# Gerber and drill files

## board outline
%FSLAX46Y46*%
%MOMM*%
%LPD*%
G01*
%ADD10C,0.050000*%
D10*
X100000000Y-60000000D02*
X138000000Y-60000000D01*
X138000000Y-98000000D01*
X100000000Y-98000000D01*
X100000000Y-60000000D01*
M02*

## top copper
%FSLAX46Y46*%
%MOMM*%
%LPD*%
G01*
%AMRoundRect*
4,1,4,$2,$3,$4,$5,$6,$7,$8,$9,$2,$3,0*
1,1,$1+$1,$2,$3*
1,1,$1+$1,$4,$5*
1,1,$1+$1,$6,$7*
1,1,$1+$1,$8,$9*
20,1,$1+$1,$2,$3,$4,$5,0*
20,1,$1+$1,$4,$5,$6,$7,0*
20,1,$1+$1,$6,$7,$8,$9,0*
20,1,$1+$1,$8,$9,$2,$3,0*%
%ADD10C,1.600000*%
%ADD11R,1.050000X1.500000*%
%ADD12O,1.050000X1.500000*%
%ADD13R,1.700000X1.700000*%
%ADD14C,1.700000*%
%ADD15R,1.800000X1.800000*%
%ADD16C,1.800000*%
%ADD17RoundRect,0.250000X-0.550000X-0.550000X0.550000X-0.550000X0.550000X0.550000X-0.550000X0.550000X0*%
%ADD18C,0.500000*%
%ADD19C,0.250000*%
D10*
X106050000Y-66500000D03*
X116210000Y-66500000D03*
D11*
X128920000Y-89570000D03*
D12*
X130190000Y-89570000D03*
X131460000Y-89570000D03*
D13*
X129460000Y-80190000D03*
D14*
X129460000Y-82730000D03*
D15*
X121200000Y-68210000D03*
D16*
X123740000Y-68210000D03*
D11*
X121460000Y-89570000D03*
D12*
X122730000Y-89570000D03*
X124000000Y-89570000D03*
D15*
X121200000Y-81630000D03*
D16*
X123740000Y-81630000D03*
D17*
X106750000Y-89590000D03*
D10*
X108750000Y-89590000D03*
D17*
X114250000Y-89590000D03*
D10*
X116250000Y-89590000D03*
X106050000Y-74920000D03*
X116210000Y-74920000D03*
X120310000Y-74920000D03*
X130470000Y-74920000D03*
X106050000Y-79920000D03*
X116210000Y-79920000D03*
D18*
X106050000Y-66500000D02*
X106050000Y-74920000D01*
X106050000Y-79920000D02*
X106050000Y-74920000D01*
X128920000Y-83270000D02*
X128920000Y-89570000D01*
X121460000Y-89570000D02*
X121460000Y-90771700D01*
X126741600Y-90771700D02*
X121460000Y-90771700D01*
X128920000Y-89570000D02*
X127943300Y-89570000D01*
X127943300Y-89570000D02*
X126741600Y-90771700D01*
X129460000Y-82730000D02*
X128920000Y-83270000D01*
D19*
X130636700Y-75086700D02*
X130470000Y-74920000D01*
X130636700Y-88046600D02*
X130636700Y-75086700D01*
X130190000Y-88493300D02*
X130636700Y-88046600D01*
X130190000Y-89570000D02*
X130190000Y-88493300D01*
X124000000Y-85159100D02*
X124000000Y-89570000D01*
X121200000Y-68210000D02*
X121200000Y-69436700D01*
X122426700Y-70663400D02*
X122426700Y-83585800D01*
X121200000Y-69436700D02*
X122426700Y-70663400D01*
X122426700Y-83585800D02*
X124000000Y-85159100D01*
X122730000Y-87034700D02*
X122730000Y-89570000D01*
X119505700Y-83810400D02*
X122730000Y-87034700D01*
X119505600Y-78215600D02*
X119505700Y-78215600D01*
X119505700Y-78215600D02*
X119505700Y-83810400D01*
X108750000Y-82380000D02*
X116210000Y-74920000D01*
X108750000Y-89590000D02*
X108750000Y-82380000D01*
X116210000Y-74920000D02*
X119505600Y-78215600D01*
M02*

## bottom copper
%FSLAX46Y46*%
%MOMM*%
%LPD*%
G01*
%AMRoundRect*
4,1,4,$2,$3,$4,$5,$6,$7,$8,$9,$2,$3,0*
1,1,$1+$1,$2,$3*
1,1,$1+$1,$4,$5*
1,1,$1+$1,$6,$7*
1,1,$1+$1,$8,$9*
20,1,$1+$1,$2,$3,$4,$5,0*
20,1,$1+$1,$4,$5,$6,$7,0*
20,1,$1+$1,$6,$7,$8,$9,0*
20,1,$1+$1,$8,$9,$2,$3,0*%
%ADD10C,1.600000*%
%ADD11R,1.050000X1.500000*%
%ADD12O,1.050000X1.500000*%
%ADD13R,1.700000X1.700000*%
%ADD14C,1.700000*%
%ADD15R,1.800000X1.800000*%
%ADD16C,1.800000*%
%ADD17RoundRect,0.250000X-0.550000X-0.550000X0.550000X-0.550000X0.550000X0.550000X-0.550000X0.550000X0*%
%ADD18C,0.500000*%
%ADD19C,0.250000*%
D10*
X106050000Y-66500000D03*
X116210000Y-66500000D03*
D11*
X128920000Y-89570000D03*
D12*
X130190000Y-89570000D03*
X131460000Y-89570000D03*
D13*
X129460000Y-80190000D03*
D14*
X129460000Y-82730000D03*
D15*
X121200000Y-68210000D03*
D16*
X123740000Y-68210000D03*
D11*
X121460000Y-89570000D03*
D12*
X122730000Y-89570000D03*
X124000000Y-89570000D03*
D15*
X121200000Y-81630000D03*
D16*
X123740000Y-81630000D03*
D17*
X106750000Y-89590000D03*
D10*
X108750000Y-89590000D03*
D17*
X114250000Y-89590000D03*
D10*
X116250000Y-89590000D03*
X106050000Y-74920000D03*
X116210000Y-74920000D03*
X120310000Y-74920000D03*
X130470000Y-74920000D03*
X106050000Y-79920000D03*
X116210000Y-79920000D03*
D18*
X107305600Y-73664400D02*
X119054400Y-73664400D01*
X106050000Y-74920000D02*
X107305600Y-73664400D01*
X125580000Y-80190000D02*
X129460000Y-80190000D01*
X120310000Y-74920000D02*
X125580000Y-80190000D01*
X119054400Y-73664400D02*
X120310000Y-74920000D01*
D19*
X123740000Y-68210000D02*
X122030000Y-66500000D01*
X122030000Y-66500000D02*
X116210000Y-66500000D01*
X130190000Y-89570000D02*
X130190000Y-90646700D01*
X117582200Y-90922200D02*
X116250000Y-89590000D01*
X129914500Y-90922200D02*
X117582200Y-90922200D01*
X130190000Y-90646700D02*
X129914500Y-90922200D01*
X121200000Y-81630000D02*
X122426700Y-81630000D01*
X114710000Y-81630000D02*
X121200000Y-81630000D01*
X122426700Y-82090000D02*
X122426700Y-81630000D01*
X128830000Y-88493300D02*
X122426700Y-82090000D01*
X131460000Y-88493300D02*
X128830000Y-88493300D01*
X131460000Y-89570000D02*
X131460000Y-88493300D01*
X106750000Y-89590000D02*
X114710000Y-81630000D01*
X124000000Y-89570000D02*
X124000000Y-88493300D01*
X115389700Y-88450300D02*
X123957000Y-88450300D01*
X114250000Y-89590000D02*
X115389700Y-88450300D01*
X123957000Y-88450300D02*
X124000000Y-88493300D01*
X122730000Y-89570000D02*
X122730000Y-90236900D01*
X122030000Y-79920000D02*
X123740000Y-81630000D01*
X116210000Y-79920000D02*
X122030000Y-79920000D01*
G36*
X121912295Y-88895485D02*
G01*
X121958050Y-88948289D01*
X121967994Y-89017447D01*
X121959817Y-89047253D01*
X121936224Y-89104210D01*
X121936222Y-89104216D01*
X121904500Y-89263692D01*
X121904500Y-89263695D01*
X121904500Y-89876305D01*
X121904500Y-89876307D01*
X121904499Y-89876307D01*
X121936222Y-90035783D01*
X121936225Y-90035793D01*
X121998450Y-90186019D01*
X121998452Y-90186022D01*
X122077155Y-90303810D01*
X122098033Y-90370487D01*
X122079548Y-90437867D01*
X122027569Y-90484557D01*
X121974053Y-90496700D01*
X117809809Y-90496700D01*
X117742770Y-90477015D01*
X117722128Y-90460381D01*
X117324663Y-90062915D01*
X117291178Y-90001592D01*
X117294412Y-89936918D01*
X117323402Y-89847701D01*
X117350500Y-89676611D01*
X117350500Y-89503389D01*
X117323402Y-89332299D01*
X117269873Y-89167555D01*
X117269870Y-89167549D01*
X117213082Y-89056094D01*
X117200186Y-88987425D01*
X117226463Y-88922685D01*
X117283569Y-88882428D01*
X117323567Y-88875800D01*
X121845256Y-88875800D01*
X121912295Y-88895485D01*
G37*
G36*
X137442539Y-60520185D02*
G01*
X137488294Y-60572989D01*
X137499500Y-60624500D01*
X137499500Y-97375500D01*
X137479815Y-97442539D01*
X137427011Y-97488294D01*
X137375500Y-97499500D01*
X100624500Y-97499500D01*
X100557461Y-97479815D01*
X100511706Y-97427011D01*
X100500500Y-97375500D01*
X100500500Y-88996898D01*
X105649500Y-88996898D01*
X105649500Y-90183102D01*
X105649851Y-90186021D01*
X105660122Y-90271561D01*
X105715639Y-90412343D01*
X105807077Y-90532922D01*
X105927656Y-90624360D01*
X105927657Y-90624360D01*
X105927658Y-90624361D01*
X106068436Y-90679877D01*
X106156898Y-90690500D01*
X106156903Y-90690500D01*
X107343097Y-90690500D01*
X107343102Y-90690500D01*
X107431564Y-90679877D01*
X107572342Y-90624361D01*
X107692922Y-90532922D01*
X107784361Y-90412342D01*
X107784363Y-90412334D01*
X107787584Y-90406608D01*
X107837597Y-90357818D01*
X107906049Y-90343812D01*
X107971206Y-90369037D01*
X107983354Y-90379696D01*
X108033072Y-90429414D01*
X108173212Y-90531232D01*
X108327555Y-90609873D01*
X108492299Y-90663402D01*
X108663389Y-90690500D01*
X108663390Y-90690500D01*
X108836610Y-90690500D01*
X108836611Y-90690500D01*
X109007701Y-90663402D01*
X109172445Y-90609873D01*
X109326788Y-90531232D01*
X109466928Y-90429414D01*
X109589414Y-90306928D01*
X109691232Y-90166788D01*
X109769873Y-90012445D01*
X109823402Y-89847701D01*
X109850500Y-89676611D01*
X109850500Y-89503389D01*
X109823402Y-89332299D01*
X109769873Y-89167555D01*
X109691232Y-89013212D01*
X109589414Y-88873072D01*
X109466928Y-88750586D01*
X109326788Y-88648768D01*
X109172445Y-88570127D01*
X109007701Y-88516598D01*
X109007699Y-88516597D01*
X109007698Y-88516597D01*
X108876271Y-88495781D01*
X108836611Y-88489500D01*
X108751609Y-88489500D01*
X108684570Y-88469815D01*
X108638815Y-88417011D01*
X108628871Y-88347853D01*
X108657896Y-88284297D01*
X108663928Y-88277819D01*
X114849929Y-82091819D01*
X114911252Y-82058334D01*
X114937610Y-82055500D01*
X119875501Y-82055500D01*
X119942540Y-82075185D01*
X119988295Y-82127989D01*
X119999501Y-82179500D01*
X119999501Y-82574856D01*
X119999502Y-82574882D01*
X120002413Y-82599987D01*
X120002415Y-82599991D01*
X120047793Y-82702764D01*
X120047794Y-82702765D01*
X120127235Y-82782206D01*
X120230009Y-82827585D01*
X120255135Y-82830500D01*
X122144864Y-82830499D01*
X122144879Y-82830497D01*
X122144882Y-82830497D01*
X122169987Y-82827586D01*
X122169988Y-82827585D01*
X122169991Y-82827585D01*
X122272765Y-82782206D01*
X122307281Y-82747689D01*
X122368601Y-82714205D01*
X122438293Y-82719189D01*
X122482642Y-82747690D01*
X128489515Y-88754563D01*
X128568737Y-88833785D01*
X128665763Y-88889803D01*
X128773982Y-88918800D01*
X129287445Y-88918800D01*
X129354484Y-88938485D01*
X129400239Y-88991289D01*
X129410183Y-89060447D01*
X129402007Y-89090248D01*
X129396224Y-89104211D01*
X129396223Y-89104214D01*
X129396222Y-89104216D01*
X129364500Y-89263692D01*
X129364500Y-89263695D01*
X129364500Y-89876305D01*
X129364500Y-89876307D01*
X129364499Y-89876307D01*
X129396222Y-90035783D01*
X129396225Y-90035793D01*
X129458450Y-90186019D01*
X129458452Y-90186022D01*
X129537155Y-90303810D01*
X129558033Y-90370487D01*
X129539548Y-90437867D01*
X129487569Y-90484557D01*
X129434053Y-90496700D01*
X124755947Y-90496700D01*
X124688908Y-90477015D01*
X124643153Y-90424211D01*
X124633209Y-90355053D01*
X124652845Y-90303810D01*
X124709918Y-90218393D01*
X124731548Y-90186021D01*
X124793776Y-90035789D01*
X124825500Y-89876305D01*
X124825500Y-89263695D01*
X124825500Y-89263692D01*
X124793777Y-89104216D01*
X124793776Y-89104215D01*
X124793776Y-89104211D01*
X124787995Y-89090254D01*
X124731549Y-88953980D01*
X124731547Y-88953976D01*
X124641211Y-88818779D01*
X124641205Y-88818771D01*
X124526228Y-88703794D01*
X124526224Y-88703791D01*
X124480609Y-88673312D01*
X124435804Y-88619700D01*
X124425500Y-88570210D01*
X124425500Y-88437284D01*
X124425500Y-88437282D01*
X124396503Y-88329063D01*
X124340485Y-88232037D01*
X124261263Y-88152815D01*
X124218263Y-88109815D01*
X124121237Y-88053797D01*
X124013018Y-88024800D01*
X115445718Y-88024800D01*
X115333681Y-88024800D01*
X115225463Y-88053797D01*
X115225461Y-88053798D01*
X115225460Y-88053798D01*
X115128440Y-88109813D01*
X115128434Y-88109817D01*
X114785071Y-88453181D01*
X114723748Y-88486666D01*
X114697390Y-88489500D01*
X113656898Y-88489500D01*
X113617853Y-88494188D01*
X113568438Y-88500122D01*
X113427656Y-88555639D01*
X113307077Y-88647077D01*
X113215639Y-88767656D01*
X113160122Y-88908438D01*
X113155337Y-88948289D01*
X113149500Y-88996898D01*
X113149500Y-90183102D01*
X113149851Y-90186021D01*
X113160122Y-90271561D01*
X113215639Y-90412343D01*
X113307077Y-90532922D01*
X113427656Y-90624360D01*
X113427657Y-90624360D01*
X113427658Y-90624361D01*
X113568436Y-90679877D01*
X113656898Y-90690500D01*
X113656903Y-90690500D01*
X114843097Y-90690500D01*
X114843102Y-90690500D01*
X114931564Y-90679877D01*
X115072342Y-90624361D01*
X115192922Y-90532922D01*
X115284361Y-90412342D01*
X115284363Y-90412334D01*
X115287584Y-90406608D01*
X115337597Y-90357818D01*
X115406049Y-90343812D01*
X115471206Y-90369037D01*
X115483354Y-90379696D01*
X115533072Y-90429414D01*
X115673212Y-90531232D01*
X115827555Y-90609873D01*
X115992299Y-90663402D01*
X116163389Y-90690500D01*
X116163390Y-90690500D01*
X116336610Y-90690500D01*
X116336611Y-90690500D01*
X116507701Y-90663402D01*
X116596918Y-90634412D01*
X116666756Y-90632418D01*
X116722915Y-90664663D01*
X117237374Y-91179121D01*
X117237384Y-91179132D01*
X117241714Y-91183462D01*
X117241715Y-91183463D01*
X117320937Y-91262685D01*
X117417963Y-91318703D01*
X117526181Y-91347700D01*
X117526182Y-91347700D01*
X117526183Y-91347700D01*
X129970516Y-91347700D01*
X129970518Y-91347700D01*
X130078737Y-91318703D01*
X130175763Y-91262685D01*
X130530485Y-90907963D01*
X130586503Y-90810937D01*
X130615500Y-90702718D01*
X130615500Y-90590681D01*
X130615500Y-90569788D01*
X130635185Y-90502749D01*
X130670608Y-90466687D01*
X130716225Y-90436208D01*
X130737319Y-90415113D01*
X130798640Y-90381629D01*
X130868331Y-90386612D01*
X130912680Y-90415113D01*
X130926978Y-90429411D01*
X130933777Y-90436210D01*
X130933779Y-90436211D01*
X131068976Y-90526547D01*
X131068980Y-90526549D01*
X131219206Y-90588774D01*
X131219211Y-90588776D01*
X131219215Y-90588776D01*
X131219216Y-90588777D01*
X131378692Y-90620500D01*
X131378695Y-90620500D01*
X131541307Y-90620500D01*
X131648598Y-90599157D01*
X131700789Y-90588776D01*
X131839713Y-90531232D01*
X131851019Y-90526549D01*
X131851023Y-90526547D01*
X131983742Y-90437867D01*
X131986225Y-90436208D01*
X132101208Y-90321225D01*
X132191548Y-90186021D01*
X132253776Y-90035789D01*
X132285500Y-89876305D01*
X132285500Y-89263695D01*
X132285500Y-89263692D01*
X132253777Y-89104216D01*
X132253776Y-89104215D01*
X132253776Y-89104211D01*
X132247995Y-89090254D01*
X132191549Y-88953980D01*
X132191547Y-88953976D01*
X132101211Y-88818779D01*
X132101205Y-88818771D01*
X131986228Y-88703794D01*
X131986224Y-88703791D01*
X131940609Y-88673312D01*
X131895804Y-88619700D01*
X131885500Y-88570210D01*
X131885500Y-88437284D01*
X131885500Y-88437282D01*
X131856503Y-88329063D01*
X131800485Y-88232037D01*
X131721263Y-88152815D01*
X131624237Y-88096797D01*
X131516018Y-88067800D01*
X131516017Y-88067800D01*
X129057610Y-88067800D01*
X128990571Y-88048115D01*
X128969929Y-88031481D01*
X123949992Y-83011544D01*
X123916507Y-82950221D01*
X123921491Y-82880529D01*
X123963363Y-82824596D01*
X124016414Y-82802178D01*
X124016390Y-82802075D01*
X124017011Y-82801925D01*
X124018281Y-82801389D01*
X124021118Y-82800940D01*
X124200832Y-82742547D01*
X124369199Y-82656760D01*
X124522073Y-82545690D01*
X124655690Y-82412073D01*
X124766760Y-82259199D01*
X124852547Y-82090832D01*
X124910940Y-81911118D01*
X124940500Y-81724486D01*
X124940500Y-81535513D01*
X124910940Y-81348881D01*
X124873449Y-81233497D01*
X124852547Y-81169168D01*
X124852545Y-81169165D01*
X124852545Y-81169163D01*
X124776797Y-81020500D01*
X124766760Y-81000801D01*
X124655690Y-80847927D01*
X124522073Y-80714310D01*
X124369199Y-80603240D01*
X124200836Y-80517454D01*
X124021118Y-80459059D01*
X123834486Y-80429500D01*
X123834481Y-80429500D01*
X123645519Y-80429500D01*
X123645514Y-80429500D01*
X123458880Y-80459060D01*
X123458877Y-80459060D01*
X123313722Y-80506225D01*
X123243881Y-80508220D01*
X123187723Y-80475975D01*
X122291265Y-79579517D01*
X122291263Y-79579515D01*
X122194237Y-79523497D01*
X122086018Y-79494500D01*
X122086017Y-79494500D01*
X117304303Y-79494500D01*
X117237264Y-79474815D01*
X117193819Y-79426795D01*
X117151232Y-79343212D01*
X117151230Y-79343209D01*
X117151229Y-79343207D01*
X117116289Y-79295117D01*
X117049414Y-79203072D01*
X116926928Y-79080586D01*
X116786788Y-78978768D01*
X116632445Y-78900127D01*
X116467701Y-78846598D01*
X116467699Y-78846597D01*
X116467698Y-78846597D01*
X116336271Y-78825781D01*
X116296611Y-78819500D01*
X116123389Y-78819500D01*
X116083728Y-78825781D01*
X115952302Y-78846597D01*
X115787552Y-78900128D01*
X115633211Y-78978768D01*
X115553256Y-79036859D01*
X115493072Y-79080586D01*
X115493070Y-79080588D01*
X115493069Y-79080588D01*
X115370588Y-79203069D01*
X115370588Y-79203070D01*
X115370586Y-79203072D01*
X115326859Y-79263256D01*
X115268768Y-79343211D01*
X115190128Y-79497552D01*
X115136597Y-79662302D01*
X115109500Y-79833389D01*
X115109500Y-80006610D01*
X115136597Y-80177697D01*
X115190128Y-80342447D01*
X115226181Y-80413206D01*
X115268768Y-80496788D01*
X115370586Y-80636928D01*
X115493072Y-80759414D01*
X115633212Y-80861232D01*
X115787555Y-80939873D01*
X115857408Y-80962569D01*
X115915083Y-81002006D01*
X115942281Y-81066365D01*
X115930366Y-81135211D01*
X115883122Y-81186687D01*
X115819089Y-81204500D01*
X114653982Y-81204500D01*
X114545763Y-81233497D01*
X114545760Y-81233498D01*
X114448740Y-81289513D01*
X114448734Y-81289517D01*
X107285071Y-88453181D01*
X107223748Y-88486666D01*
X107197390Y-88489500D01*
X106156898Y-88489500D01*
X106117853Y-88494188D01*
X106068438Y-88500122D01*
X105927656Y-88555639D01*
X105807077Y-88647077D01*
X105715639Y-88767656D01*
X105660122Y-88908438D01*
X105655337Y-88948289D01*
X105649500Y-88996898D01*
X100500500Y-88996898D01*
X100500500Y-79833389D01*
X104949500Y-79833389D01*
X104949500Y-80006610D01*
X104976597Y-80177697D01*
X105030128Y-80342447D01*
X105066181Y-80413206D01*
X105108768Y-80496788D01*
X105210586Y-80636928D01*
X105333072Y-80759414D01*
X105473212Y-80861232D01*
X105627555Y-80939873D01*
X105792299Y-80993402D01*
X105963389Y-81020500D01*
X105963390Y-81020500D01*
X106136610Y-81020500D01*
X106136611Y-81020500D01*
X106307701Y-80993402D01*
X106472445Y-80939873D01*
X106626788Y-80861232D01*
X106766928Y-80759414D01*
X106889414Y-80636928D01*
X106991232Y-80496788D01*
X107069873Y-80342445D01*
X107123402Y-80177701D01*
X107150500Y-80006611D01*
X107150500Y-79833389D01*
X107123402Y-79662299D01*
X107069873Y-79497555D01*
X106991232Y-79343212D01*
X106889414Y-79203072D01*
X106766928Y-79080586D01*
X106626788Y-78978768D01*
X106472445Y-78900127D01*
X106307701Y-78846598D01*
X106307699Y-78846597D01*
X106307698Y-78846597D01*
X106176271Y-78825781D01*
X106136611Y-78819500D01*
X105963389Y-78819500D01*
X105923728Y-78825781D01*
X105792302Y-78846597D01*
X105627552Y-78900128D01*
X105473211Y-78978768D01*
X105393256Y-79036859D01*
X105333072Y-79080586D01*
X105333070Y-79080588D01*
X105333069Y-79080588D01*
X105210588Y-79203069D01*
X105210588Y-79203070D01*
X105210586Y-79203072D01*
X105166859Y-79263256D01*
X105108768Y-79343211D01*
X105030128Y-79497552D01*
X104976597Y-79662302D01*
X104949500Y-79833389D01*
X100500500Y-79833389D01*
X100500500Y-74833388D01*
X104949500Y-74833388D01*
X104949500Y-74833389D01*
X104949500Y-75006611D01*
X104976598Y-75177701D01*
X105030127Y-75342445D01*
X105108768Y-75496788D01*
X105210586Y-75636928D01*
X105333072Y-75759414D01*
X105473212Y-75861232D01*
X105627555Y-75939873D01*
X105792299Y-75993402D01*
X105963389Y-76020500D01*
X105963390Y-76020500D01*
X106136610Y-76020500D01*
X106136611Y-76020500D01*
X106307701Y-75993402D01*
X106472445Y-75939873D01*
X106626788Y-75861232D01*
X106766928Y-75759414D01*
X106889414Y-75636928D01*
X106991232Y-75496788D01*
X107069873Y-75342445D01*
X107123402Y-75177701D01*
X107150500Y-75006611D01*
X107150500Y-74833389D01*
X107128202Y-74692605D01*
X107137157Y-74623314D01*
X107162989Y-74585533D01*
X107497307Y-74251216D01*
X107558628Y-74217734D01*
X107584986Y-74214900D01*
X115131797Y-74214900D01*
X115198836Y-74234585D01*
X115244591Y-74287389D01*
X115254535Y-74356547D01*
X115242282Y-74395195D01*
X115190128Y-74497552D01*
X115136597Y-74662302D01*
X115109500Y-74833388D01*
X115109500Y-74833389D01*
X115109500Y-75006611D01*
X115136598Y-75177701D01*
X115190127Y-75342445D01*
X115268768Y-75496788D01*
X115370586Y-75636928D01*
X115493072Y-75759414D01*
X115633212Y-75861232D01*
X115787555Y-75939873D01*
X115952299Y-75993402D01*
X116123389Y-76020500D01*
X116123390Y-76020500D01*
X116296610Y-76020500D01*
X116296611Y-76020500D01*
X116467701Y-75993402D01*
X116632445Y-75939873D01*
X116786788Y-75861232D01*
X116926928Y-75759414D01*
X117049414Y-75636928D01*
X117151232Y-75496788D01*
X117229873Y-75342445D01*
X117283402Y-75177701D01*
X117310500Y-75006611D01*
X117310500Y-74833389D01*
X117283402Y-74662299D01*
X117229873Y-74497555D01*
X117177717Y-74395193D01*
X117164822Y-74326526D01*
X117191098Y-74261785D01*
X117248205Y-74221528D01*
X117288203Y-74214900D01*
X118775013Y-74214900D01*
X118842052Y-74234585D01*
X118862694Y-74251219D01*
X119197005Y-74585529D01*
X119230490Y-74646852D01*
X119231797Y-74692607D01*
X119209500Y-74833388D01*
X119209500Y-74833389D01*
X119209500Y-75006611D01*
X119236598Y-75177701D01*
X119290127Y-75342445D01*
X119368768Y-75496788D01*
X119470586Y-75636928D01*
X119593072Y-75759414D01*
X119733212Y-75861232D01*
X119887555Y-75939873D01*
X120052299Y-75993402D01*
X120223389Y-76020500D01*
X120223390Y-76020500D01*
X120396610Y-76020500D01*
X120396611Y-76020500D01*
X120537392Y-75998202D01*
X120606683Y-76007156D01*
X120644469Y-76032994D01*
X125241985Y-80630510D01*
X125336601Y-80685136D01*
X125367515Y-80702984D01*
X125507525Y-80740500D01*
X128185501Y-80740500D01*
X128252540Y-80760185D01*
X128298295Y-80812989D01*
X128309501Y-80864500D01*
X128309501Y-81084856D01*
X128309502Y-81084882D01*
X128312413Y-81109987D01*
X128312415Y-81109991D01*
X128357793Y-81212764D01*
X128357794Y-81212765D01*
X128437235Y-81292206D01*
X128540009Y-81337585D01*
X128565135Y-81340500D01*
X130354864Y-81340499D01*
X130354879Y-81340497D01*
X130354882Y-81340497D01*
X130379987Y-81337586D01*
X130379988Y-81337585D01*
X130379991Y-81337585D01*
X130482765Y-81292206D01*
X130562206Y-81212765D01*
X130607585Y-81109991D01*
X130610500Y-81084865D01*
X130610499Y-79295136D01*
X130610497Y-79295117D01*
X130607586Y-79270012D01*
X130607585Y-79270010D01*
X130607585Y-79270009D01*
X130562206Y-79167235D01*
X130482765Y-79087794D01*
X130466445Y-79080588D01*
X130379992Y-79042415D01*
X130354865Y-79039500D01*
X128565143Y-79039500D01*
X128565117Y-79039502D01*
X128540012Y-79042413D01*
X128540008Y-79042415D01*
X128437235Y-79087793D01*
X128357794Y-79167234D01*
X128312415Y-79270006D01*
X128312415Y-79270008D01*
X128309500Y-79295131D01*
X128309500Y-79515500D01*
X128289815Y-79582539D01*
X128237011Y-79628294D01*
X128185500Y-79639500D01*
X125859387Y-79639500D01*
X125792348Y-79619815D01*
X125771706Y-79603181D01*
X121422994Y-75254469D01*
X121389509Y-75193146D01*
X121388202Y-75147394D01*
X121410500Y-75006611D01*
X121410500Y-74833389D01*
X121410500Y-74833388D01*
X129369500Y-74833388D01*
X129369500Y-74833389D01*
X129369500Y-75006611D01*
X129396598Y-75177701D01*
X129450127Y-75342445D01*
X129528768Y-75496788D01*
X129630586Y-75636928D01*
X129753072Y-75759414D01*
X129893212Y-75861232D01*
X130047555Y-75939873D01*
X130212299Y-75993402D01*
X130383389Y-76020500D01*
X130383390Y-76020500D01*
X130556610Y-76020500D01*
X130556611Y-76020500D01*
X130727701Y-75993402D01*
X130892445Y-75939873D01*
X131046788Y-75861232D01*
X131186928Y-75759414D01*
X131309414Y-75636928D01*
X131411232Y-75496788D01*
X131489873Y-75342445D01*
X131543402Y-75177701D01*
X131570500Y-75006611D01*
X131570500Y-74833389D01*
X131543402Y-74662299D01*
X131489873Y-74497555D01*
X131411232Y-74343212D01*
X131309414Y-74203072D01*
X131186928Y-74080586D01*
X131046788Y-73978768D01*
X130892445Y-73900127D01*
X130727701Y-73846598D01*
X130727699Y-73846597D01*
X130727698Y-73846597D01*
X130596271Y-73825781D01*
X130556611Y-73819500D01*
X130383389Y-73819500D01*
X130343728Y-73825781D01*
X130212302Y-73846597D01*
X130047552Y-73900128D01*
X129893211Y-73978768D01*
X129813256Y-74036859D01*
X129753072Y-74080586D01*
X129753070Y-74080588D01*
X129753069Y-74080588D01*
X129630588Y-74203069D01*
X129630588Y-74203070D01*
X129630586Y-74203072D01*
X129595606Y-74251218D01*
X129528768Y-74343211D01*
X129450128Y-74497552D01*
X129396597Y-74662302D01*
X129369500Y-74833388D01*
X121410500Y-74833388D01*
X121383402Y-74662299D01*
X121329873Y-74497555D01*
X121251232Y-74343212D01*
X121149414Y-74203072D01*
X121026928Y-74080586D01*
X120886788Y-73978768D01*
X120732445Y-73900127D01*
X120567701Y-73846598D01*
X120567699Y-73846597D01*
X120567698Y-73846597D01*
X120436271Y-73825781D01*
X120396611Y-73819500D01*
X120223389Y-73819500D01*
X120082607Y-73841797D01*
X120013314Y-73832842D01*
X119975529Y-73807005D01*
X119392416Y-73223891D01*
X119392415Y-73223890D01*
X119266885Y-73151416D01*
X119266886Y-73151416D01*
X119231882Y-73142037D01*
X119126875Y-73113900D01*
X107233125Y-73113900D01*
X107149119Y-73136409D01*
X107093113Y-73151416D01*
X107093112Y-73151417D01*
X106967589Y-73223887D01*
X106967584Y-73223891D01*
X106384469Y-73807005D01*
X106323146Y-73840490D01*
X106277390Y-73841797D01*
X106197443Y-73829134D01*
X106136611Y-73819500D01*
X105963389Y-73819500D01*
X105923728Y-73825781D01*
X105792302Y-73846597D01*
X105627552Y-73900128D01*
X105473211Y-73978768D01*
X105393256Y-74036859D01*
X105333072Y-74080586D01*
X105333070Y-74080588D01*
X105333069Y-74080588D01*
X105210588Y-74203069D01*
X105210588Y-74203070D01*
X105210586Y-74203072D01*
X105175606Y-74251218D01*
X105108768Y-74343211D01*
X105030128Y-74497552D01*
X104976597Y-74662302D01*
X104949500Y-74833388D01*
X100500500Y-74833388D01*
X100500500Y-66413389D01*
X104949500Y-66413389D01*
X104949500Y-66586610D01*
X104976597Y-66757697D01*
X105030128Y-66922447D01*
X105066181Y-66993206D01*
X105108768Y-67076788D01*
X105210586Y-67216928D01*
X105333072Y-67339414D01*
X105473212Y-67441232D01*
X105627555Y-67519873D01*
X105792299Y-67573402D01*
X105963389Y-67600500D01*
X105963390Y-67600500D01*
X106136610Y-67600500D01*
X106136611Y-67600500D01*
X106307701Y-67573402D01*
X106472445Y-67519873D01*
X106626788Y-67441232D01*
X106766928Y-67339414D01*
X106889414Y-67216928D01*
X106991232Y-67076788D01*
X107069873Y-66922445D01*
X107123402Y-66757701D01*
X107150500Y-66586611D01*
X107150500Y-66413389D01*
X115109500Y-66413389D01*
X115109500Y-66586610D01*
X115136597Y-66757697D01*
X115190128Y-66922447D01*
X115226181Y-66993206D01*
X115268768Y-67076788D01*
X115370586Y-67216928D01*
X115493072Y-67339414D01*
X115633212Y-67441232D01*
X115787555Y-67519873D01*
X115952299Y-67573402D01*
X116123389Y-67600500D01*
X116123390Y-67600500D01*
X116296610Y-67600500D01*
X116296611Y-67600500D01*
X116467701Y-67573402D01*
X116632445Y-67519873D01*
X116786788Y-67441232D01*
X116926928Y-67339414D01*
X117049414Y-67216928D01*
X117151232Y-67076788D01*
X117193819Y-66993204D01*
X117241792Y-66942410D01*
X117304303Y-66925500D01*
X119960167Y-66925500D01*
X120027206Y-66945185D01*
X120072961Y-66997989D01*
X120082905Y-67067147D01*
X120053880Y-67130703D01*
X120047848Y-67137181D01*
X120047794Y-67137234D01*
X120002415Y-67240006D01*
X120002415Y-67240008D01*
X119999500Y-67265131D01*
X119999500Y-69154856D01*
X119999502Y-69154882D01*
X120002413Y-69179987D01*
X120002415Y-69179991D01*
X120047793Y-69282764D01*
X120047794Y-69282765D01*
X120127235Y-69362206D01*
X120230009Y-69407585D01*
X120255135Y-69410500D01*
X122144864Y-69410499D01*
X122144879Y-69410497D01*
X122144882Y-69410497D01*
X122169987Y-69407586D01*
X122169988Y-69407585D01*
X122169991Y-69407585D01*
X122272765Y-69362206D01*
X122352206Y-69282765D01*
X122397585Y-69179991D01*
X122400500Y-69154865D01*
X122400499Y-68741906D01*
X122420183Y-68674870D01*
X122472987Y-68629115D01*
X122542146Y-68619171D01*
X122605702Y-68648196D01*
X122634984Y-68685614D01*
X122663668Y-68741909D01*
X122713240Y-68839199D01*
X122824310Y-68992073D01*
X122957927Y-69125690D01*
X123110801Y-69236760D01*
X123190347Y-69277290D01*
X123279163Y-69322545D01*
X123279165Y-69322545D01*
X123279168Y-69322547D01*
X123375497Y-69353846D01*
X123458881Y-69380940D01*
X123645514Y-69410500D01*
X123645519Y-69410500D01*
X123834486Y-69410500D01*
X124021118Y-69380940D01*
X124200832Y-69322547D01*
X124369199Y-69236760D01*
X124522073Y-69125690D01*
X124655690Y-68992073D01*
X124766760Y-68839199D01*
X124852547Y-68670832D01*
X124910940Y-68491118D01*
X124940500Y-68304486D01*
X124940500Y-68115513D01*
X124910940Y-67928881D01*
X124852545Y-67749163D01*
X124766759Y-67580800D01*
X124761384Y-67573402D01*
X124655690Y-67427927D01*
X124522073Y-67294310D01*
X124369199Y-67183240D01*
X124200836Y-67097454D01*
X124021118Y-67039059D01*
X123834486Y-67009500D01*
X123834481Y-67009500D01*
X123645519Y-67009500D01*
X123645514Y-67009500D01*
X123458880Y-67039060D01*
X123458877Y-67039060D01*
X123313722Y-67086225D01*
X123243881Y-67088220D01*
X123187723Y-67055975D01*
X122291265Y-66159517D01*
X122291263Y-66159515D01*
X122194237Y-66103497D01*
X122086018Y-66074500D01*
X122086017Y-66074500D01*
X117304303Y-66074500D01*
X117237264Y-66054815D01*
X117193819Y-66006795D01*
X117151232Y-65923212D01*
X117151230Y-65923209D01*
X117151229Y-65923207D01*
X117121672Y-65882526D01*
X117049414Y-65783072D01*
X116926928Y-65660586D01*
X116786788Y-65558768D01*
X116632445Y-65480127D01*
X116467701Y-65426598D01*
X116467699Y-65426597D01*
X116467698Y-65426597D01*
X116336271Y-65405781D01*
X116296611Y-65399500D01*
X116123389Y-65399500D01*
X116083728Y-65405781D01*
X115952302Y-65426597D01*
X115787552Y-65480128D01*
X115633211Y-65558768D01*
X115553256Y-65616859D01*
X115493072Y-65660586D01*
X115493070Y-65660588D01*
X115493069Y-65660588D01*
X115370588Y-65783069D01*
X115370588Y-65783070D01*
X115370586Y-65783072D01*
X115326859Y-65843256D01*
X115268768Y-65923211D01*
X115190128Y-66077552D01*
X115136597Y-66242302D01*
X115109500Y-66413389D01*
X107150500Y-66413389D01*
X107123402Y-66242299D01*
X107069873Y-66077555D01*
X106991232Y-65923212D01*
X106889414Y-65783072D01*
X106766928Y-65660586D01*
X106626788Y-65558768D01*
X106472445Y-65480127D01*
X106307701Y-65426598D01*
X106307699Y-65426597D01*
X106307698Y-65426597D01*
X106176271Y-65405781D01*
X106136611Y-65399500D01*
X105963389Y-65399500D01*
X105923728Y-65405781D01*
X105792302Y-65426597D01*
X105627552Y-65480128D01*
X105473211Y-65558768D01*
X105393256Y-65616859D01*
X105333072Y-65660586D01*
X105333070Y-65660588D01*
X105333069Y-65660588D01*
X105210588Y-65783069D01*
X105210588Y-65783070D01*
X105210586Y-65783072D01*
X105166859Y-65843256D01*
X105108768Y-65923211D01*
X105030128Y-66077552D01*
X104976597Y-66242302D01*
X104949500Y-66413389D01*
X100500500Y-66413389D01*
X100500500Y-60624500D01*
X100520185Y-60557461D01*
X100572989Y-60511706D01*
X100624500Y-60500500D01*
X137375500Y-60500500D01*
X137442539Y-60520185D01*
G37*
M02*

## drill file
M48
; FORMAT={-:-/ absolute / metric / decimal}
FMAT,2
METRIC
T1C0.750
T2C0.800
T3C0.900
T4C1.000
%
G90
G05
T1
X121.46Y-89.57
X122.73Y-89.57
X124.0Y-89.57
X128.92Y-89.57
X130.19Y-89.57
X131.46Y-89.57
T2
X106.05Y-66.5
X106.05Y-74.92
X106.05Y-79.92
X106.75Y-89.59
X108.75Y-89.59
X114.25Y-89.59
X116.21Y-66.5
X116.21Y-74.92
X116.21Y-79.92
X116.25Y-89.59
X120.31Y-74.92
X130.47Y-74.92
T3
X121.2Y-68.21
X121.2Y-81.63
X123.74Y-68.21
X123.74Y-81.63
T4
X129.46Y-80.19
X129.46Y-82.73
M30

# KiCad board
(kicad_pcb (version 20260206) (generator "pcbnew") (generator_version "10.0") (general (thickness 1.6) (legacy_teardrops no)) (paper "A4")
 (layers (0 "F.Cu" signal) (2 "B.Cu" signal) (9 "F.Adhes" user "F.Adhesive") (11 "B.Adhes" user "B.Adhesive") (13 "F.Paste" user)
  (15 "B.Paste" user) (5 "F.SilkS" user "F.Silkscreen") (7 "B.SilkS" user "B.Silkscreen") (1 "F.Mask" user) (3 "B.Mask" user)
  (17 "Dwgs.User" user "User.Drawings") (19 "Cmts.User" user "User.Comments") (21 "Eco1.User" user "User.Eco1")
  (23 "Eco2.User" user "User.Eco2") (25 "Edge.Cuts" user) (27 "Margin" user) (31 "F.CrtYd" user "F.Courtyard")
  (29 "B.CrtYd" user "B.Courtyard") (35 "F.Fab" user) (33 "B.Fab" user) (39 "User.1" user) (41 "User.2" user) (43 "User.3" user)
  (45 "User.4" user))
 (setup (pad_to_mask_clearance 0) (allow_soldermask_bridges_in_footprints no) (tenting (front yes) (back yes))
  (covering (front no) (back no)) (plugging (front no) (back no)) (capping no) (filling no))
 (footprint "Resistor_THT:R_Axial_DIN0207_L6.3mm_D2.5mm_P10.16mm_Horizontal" (layer "F.Cu") (at 106.05 66.5)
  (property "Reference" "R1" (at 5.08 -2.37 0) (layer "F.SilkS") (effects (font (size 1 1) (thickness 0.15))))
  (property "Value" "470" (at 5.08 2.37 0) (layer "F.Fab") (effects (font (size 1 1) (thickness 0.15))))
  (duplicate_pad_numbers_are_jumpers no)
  (pad "1" thru_hole circle (at 0 0) (size 1.6 1.6) (drill 0.8) (layers "*.Cu" "*.Mask") (remove_unused_layers no) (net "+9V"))
  (pad "2" thru_hole circle (at 10.16 0) (size 1.6 1.6) (drill 0.8) (layers "*.Cu" "*.Mask") (remove_unused_layers no)
   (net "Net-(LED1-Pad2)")))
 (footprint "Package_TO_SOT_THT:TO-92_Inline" (layer "F.Cu") (at 128.92 89.57)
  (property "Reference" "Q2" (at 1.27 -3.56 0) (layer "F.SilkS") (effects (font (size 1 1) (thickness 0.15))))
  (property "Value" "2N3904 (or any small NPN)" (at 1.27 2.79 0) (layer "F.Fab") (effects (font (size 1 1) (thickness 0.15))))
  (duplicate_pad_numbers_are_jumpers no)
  (pad "1" thru_hole rect (at 0 0) (size 1.05 1.5) (drill 0.75) (layers "*.Cu" "*.Mask") (remove_unused_layers no) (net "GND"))
  (pad "2" thru_hole oval (at 1.27 0) (size 1.05 1.5) (drill 0.75) (layers "*.Cu" "*.Mask") (remove_unused_layers no) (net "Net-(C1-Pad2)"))
  (pad "3" thru_hole oval (at 2.54 0) (size 1.05 1.5) (drill 0.75) (layers "*.Cu" "*.Mask") (remove_unused_layers no) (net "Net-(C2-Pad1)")))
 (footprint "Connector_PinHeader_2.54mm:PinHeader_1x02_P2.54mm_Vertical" (layer "F.Cu") (at 129.46 80.19)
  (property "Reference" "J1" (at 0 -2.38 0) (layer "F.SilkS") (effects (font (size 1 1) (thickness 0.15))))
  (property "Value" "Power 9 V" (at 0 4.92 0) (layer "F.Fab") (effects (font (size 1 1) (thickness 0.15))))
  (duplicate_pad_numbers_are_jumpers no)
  (pad "1" thru_hole rect (at 0 0) (size 1.7 1.7) (drill 1) (layers "*.Cu" "*.Mask") (remove_unused_layers no) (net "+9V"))
  (pad "2" thru_hole circle (at 0 2.54) (size 1.7 1.7) (drill 1) (layers "*.Cu" "*.Mask") (remove_unused_layers no) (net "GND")))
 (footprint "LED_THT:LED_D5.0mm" (layer "F.Cu") (at 121.2 68.21)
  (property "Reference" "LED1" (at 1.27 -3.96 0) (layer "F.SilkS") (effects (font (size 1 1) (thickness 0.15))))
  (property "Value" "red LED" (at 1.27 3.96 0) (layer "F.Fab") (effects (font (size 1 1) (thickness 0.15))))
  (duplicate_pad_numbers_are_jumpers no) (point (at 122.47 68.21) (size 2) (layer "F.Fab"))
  (pad "1" thru_hole rect (at 0 0) (size 1.8 1.8) (drill 0.9) (layers "*.Cu" "*.Mask") (remove_unused_layers no) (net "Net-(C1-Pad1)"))
  (pad "2" thru_hole circle (at 2.54 0) (size 1.8 1.8) (drill 0.9) (layers "*.Cu" "*.Mask") (remove_unused_layers no)
   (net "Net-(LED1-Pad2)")))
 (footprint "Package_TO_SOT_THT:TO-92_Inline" (layer "F.Cu") (at 121.46 89.57)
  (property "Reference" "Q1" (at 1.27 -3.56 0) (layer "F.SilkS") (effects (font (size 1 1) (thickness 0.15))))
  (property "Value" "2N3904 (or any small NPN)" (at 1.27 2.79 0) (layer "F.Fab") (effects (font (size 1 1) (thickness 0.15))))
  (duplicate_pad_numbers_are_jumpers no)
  (pad "1" thru_hole rect (at 0 0) (size 1.05 1.5) (drill 0.75) (layers "*.Cu" "*.Mask") (remove_unused_layers no) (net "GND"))
  (pad "2" thru_hole oval (at 1.27 0) (size 1.05 1.5) (drill 0.75) (layers "*.Cu" "*.Mask") (remove_unused_layers no) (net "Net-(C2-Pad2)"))
  (pad "3" thru_hole oval (at 2.54 0) (size 1.05 1.5) (drill 0.75) (layers "*.Cu" "*.Mask") (remove_unused_layers no) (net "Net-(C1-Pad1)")))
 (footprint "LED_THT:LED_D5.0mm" (layer "F.Cu") (at 121.2 81.63)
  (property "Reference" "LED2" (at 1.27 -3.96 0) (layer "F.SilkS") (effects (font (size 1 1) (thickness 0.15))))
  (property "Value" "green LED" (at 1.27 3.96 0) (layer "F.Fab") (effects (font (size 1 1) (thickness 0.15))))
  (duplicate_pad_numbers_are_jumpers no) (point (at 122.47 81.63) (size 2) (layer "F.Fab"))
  (pad "1" thru_hole rect (at 0 0) (size 1.8 1.8) (drill 0.9) (layers "*.Cu" "*.Mask") (remove_unused_layers no) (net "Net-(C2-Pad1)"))
  (pad "2" thru_hole circle (at 2.54 0) (size 1.8 1.8) (drill 0.9) (layers "*.Cu" "*.Mask") (remove_unused_layers no)
   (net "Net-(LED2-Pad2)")))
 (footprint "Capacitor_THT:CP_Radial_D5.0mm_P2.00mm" (layer "F.Cu") (at 106.75 89.59)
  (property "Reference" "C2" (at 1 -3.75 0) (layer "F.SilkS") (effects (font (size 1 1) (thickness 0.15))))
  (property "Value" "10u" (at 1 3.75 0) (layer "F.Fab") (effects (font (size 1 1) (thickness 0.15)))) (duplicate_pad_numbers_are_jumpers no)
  (pad "1" thru_hole roundrect (at 0 0) (size 1.6 1.6) (drill 0.8) (layers "*.Cu" "*.Mask") (remove_unused_layers no)
   (roundrect_rratio 0.15625) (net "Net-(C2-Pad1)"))
  (pad "2" thru_hole circle (at 2 0) (size 1.6 1.6) (drill 0.8) (layers "*.Cu" "*.Mask") (remove_unused_layers no) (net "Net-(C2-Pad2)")))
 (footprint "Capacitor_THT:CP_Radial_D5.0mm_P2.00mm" (layer "F.Cu") (at 114.25 89.59)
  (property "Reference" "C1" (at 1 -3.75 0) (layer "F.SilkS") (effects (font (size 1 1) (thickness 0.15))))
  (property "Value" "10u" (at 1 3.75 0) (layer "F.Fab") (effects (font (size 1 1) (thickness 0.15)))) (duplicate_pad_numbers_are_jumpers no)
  (pad "1" thru_hole roundrect (at 0 0) (size 1.6 1.6) (drill 0.8) (layers "*.Cu" "*.Mask") (remove_unused_layers no)
   (roundrect_rratio 0.15625) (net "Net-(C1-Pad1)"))
  (pad "2" thru_hole circle (at 2 0) (size 1.6 1.6) (drill 0.8) (layers "*.Cu" "*.Mask") (remove_unused_layers no) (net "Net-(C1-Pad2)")))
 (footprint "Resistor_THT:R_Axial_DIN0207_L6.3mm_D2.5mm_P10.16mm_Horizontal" (layer "F.Cu") (at 106.05 74.92)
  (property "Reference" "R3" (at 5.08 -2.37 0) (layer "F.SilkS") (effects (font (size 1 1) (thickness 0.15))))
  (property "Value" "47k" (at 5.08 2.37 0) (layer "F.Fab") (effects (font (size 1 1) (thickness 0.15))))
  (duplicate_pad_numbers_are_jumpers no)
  (pad "1" thru_hole circle (at 0 0) (size 1.6 1.6) (drill 0.8) (layers "*.Cu" "*.Mask") (remove_unused_layers no) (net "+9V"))
  (pad "2" thru_hole circle (at 10.16 0) (size 1.6 1.6) (drill 0.8) (layers "*.Cu" "*.Mask") (remove_unused_layers no) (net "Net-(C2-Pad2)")))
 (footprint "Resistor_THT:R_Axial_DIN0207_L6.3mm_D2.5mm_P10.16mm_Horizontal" (layer "F.Cu") (at 120.31 74.92)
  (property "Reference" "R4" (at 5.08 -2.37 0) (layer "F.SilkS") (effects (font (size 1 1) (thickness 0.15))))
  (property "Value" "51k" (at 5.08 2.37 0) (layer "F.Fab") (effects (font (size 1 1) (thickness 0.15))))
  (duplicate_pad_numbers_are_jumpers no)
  (pad "1" thru_hole circle (at 0 0) (size 1.6 1.6) (drill 0.8) (layers "*.Cu" "*.Mask") (remove_unused_layers no) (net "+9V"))
  (pad "2" thru_hole circle (at 10.16 0) (size 1.6 1.6) (drill 0.8) (layers "*.Cu" "*.Mask") (remove_unused_layers no) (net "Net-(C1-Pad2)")))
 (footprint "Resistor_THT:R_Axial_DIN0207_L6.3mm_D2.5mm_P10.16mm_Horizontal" (layer "F.Cu") (at 106.05 79.92)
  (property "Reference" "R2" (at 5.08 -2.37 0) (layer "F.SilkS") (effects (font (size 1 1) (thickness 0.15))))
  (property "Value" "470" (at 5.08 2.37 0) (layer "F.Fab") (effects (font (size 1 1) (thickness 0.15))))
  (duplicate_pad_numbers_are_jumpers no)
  (pad "1" thru_hole circle (at 0 0) (size 1.6 1.6) (drill 0.8) (layers "*.Cu" "*.Mask") (remove_unused_layers no) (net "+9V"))
  (pad "2" thru_hole circle (at 10.16 0) (size 1.6 1.6) (drill 0.8) (layers "*.Cu" "*.Mask") (remove_unused_layers no)
   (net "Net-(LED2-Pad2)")))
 (gr_rect (start 100 60) (end 138 98) (stroke (width 0.05) (type default)) (fill no) (layer "Edge.Cuts"))
 (segment (start 106.05 66.5) (end 106.05 74.92) (width 0.5) (layer "F.Cu") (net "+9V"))
 (segment (start 106.05 79.92) (end 106.05 74.92) (width 0.5) (layer "F.Cu") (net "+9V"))
 (segment (start 107.3056 73.6644) (end 119.0544 73.6644) (width 0.5) (layer "B.Cu") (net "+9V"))
 (segment (start 106.05 74.92) (end 107.3056 73.6644) (width 0.5) (layer "B.Cu") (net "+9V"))
 (segment (start 125.58 80.19) (end 129.46 80.19) (width 0.5) (layer "B.Cu") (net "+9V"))
 (segment (start 120.31 74.92) (end 125.58 80.19) (width 0.5) (layer "B.Cu") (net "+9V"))
 (segment (start 119.0544 73.6644) (end 120.31 74.92) (width 0.5) (layer "B.Cu") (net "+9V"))
 (segment (start 123.74 68.21) (end 122.03 66.5) (width 0.25) (layer "B.Cu") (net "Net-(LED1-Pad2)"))
 (segment (start 122.03 66.5) (end 116.21 66.5) (width 0.25) (layer "B.Cu") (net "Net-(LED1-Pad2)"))
 (segment (start 128.92 83.27) (end 128.92 89.57) (width 0.5) (layer "F.Cu") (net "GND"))
 (segment (start 121.46 89.57) (end 121.46 90.7717) (width 0.5) (layer "F.Cu") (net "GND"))
 (segment (start 126.7416 90.7717) (end 121.46 90.7717) (width 0.5) (layer "F.Cu") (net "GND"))
 (segment (start 128.92 89.57) (end 127.9433 89.57) (width 0.5) (layer "F.Cu") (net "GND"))
 (segment (start 127.9433 89.57) (end 126.7416 90.7717) (width 0.5) (layer "F.Cu") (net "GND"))
 (segment (start 129.46 82.73) (end 128.92 83.27) (width 0.5) (layer "F.Cu") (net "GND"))
 (segment (start 130.6367 75.0867) (end 130.47 74.92) (width 0.25) (layer "F.Cu") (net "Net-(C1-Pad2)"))
 (segment (start 130.6367 88.0466) (end 130.6367 75.0867) (width 0.25) (layer "F.Cu") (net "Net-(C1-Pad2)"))
 (segment (start 130.19 88.4933) (end 130.6367 88.0466) (width 0.25) (layer "F.Cu") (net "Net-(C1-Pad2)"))
 (segment (start 130.19 89.57) (end 130.19 88.4933) (width 0.25) (layer "F.Cu") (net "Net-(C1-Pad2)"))
 (segment (start 130.19 89.57) (end 130.19 90.6467) (width 0.25) (layer "B.Cu") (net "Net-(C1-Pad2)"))
 (segment (start 117.5822 90.9222) (end 116.25 89.59) (width 0.25) (layer "B.Cu") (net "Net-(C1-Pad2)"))
 (segment (start 129.9145 90.9222) (end 117.5822 90.9222) (width 0.25) (layer "B.Cu") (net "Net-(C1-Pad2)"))
 (segment (start 130.19 90.6467) (end 129.9145 90.9222) (width 0.25) (layer "B.Cu") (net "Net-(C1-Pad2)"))
 (segment (start 121.2 81.63) (end 122.4267 81.63) (width 0.25) (layer "B.Cu") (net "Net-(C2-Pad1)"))
 (segment (start 114.71 81.63) (end 121.2 81.63) (width 0.25) (layer "B.Cu") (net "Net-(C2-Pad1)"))
 (segment (start 122.4267 82.09) (end 122.4267 81.63) (width 0.25) (layer "B.Cu") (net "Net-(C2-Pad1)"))
 (segment (start 128.83 88.4933) (end 122.4267 82.09) (width 0.25) (layer "B.Cu") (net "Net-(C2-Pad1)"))
 (segment (start 131.46 88.4933) (end 128.83 88.4933) (width 0.25) (layer "B.Cu") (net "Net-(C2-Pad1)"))
 (segment (start 131.46 89.57) (end 131.46 88.4933) (width 0.25) (layer "B.Cu") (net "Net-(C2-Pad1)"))
 (segment (start 106.75 89.59) (end 114.71 81.63) (width 0.25) (layer "B.Cu") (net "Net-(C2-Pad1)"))
 (segment (start 124 85.1591) (end 124 89.57) (width 0.25) (layer "F.Cu") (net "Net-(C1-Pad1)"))
 (segment (start 121.2 68.21) (end 121.2 69.4367) (width 0.25) (layer "F.Cu") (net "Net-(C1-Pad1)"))
 (segment (start 122.4267 70.6634) (end 122.4267 83.5858) (width 0.25) (layer "F.Cu") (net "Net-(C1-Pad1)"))
 (segment (start 121.2 69.4367) (end 122.4267 70.6634) (width 0.25) (layer "F.Cu") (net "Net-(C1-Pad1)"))
 (segment (start 122.4267 83.5858) (end 124 85.1591) (width 0.25) (layer "F.Cu") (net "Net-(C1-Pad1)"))
 (segment (start 124 89.57) (end 124 88.4933) (width 0.25) (layer "B.Cu") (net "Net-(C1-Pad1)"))
 (segment (start 115.3897 88.4503) (end 123.957 88.4503) (width 0.25) (layer "B.Cu") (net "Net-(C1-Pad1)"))
 (segment (start 114.25 89.59) (end 115.3897 88.4503) (width 0.25) (layer "B.Cu") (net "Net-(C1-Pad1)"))
 (segment (start 123.957 88.4503) (end 124 88.4933) (width 0.25) (layer "B.Cu") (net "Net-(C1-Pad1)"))
 (segment (start 122.73 87.0347) (end 122.73 89.57) (width 0.25) (layer "F.Cu") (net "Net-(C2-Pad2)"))
 (segment (start 119.5057 83.8104) (end 122.73 87.0347) (width 0.25) (layer "F.Cu") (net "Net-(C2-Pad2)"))
 (segment (start 119.5056 78.2156) (end 119.5057 78.2156) (width 0.25) (layer "F.Cu") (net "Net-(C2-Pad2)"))
 (segment (start 119.5057 78.2156) (end 119.5057 83.8104) (width 0.25) (layer "F.Cu") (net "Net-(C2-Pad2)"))
 (segment (start 108.75 82.38) (end 116.21 74.92) (width 0.25) (layer "F.Cu") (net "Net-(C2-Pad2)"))
 (segment (start 108.75 89.59) (end 108.75 82.38) (width 0.25) (layer "F.Cu") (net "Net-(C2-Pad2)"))
 (segment (start 116.21 74.92) (end 119.5056 78.2156) (width 0.25) (layer "F.Cu") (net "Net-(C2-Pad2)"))
 (segment (start 122.73 89.57) (end 122.73 90.2369) (width 0.25) (layer "B.Cu") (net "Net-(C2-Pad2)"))
 (segment (start 122.03 79.92) (end 123.74 81.63) (width 0.25) (layer "B.Cu") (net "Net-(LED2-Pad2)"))
 (segment (start 116.21 79.92) (end 122.03 79.92) (width 0.25) (layer "B.Cu") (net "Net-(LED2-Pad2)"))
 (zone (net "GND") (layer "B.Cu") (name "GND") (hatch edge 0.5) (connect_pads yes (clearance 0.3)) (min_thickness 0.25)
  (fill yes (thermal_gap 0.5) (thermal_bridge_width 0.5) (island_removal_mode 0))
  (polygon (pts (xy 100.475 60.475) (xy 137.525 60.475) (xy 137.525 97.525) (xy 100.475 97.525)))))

